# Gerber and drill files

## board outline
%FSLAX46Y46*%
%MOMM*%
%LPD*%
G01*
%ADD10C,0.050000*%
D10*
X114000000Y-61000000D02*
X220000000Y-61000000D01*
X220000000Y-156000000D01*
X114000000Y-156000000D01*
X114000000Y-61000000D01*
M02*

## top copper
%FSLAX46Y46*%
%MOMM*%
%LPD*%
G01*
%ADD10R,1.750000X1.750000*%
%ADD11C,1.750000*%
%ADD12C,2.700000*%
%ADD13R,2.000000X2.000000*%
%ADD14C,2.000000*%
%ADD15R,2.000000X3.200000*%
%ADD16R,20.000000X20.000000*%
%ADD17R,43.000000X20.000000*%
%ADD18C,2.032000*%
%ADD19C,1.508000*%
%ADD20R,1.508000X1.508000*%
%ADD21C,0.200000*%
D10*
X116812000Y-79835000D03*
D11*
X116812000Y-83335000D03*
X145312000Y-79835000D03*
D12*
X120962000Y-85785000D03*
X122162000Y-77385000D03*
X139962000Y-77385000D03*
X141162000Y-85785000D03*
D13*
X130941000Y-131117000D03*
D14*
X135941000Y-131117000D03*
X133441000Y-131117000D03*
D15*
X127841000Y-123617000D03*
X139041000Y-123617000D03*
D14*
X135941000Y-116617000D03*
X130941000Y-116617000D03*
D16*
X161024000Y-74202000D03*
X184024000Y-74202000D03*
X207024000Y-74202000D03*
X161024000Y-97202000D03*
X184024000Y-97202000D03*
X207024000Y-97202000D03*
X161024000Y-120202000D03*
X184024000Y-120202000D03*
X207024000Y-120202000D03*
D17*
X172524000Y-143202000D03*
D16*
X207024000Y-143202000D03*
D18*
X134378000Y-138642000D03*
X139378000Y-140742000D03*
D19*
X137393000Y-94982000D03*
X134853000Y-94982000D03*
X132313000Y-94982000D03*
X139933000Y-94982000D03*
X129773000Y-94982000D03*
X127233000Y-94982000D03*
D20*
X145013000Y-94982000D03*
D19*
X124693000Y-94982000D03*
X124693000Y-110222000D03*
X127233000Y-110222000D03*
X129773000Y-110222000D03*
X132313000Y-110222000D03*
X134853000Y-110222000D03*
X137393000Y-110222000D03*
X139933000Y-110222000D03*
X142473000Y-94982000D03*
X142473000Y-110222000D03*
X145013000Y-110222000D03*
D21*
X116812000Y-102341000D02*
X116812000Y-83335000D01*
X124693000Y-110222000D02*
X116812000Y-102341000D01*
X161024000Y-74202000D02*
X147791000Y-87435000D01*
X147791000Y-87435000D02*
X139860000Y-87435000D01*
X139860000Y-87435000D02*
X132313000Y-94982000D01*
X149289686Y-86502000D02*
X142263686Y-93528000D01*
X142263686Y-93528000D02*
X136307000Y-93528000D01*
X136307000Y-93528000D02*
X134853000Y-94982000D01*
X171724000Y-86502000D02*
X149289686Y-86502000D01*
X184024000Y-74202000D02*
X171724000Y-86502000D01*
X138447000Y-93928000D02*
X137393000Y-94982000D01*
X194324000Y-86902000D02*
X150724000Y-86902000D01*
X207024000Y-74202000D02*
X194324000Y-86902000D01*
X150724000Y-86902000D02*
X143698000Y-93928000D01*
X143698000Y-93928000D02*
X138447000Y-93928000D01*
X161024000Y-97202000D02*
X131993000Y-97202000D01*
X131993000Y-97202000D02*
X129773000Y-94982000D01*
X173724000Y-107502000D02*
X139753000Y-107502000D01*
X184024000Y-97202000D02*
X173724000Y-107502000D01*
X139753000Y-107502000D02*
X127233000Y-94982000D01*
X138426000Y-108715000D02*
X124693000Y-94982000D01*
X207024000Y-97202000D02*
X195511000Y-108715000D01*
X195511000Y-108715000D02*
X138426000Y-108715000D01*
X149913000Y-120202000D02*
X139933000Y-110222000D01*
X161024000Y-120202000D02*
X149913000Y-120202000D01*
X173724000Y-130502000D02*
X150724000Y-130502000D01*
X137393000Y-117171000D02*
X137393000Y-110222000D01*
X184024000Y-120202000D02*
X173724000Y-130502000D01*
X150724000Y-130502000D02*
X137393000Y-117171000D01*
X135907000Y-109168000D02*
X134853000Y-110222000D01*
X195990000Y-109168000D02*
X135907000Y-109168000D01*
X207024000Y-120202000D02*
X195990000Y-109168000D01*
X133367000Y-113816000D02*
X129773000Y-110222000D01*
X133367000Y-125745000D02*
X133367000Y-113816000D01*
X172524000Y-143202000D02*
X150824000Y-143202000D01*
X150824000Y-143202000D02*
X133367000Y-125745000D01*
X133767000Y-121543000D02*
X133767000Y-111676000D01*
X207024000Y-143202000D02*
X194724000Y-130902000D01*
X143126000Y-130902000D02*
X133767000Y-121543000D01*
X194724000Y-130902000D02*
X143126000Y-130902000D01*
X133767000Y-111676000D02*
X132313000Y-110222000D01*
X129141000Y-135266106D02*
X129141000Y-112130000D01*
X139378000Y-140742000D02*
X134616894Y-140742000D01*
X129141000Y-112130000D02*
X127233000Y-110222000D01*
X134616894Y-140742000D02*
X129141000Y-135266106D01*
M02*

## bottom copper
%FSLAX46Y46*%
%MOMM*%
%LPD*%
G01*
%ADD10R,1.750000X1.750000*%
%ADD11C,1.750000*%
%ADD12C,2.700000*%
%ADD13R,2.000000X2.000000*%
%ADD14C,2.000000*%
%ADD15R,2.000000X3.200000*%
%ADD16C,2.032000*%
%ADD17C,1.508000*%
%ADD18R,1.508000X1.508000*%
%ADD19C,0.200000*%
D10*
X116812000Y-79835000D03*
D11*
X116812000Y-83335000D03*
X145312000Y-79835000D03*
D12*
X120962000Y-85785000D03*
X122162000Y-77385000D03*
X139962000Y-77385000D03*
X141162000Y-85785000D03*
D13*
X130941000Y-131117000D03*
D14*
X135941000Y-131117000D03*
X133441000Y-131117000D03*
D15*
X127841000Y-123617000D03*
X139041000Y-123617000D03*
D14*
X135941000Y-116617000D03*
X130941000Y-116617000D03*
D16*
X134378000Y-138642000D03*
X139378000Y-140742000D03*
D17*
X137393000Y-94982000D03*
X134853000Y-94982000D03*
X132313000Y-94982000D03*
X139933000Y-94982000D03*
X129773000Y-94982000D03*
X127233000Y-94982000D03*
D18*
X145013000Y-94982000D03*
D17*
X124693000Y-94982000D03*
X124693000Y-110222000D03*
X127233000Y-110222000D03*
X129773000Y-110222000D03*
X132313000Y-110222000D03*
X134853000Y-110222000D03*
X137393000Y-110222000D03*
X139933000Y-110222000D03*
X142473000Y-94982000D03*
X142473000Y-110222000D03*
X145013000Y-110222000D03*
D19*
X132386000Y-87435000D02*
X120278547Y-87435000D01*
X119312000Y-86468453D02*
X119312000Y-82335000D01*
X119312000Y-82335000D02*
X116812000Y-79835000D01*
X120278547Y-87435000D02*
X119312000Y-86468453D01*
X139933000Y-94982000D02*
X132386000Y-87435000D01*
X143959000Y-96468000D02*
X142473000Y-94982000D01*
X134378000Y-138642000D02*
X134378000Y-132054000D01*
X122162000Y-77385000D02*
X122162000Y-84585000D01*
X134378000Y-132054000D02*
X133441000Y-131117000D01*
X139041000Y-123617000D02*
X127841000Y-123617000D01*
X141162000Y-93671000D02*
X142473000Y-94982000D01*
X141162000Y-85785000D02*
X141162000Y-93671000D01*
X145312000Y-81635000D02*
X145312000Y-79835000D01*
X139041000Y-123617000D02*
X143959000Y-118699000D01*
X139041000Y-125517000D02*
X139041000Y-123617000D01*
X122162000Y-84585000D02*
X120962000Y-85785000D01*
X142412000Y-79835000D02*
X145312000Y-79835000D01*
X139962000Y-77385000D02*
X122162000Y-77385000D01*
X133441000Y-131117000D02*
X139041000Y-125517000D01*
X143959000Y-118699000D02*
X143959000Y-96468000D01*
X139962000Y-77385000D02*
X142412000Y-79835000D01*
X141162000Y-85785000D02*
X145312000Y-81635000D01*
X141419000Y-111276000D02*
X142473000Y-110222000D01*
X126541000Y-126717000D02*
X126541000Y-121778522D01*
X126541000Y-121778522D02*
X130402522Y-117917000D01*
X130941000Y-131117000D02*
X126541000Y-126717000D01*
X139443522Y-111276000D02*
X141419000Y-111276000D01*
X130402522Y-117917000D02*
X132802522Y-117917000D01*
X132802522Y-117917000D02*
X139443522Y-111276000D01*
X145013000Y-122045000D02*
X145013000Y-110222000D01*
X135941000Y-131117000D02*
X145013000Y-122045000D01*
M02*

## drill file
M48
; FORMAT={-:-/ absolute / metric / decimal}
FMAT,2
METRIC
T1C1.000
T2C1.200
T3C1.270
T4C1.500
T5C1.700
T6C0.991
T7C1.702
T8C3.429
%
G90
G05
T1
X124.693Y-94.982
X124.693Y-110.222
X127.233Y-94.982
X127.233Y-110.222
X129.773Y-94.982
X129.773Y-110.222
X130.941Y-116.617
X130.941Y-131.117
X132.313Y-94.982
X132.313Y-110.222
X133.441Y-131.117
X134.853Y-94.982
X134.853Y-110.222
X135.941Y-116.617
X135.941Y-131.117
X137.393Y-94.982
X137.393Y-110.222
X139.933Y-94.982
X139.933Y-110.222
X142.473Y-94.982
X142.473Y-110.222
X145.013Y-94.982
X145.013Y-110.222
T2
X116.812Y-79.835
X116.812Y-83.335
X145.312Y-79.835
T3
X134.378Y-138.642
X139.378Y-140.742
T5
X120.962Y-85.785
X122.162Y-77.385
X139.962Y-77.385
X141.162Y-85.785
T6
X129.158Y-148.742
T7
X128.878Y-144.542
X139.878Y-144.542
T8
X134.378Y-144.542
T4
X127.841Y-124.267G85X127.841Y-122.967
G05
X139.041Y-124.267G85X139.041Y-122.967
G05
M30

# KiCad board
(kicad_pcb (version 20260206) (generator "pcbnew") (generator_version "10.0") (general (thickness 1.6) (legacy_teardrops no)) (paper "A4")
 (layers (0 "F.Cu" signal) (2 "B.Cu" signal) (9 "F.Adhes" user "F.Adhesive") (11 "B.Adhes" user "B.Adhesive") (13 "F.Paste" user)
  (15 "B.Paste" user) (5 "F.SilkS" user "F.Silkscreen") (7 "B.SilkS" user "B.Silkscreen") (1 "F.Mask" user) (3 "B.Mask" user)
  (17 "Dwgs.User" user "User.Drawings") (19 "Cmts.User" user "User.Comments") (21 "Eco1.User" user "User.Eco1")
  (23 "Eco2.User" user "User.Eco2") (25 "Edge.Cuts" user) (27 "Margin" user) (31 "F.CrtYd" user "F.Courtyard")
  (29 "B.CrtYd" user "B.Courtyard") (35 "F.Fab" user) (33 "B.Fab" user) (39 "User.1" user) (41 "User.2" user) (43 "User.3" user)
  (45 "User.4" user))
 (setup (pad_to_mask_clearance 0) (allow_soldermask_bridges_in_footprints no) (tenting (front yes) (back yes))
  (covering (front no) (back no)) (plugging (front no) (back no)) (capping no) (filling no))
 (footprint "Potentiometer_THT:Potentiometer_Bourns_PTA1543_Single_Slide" (layer "F.Cu") (at 116.812 79.835)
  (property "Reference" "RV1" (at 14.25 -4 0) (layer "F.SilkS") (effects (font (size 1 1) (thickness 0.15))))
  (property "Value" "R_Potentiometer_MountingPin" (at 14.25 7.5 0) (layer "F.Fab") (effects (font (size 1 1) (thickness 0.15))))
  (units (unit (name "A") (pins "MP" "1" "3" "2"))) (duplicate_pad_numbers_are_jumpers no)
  (pad "1" thru_hole rect (at 0 0) (size 1.75 1.75) (drill 1.2) (layers "*.Cu" "*.Mask") (remove_unused_layers no) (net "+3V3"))
  (pad "2" thru_hole circle (at 0 3.5) (size 1.75 1.75) (drill 1.2) (layers "*.Cu" "*.Mask") (remove_unused_layers no) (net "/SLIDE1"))
  (pad "3" thru_hole circle (at 28.5 0) (size 1.75 1.75) (drill 1.2) (layers "*.Cu" "*.Mask") (remove_unused_layers no) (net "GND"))
  (pad "MP" thru_hole circle (at 4.15 5.95) (size 2.7 2.7) (drill 1.7) (layers "*.Cu" "*.Mask") (remove_unused_layers no) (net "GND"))
  (pad "MP" thru_hole circle (at 5.35 -2.45) (size 2.7 2.7) (drill 1.7) (layers "*.Cu" "*.Mask") (remove_unused_layers no) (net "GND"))
  (pad "MP" thru_hole circle (at 23.15 -2.45) (size 2.7 2.7) (drill 1.7) (layers "*.Cu" "*.Mask") (remove_unused_layers no) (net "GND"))
  (pad "MP" thru_hole circle (at 24.35 5.95) (size 2.7 2.7) (drill 1.7) (layers "*.Cu" "*.Mask") (remove_unused_layers no) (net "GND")))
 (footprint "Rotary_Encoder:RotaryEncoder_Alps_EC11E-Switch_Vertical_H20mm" (layer "F.Cu") (at 130.941 131.117 90)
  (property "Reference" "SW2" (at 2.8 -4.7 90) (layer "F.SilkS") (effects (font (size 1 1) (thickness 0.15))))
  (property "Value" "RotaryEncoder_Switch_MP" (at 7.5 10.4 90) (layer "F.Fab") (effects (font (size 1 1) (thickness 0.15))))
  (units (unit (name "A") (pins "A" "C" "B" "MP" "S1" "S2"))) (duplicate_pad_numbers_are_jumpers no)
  (pad "A" thru_hole rect (at 0 0 90) (size 2 2) (drill 1) (layers "*.Cu" "*.Mask") (remove_unused_layers no) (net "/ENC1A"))
  (pad "B" thru_hole circle (at 0 5 90) (size 2 2) (drill 1) (layers "*.Cu" "*.Mask") (remove_unused_layers no) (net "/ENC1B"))
  (pad "C" thru_hole circle (at 0 2.5 90) (size 2 2) (drill 1) (layers "*.Cu" "*.Mask") (remove_unused_layers no) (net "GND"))
  (pad "MP" thru_hole rect (at 7.5 -3.1 90) (size 3.2 2) (drill oval 2.8 1.5) (layers "*.Cu" "*.Mask") (remove_unused_layers no) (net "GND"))
  (pad "MP" thru_hole rect (at 7.5 8.1 90) (size 3.2 2) (drill oval 2.8 1.5) (layers "*.Cu" "*.Mask") (remove_unused_layers no) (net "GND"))
  (pad "S1" thru_hole circle (at 14.5 5 90) (size 2 2) (drill 1) (layers "*.Cu" "*.Mask") (remove_unused_layers no)
   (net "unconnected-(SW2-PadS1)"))
  (pad "S2" thru_hole circle (at 14.5 0 90) (size 2 2) (drill 1) (layers "*.Cu" "*.Mask") (remove_unused_layers no)
   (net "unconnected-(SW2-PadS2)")))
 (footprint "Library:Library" (layer "F.Cu") (at 180.024 57.202)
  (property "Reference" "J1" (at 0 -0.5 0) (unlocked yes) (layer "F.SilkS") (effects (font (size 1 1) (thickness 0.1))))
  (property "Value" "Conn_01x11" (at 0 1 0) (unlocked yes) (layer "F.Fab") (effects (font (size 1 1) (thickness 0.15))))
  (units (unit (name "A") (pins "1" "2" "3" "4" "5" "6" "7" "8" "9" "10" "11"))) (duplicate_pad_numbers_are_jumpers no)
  (pad "1" smd rect (at -19 17) (size 20 20) (layers "F.Cu" "F.Mask") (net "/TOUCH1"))
  (pad "2" smd rect (at 4 17) (size 20 20) (layers "F.Cu" "F.Mask") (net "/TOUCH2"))
  (pad "3" smd rect (at 27 17) (size 20 20) (layers "F.Cu" "F.Mask") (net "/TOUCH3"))
  (pad "4" smd rect (at -19 40) (size 20 20) (layers "F.Cu" "F.Mask") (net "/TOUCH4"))
  (pad "5" smd rect (at 4 40) (size 20 20) (layers "F.Cu" "F.Mask") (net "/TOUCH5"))
  (pad "6" smd rect (at 27 40) (size 20 20) (layers "F.Cu" "F.Mask") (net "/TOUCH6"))
  (pad "7" smd rect (at -19 63) (size 20 20) (layers "F.Cu" "F.Mask") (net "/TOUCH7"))
  (pad "8" smd rect (at 4 63) (size 20 20) (layers "F.Cu" "F.Mask") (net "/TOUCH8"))
  (pad "9" smd rect (at 27 63) (size 20 20) (layers "F.Cu" "F.Mask") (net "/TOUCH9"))
  (pad "10" smd rect (at -7.5 86) (size 43 20) (layers "F.Cu" "F.Mask") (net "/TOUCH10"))
  (pad "11" smd rect (at 27 86) (size 20 20) (layers "F.Cu" "F.Mask") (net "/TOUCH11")))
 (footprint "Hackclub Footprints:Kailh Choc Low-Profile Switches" (layer "F.Cu") (at 134.378 144.542 180)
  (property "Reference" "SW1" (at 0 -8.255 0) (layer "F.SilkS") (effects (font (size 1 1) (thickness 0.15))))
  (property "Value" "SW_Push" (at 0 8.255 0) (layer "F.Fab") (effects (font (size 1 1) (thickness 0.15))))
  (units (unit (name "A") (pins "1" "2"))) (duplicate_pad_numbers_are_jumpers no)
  (pad "" np_thru_hole circle (at -5.5 0 180) (size 1.7018 1.7018) (drill 1.7018) (layers "*.Cu" "*.Mask"))
  (pad "" np_thru_hole circle (at 0 0 180) (size 3.429 3.429) (drill 3.429) (layers "*.Cu" "*.Mask"))
  (pad "" np_thru_hole circle (at 5.22 -4.2 180) (size 0.9906 0.9906) (drill 0.9906) (layers "*.Cu" "*.Mask"))
  (pad "" np_thru_hole circle (at 5.5 0 180) (size 1.7018 1.7018) (drill 1.7018) (layers "*.Cu" "*.Mask"))
  (pad "1" thru_hole circle (at 0 5.9 180) (size 2.032 2.032) (drill 1.27) (layers "*.Cu" "*.Mask") (remove_unused_layers no) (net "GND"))
  (pad "2" thru_hole circle (at -5 3.8 180) (size 2.032 2.032) (drill 1.27) (layers "*.Cu" "*.Mask") (remove_unused_layers no)
   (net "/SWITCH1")))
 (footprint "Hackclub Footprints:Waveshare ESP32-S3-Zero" (layer "F.Cu") (at 134.853 102.602 -90)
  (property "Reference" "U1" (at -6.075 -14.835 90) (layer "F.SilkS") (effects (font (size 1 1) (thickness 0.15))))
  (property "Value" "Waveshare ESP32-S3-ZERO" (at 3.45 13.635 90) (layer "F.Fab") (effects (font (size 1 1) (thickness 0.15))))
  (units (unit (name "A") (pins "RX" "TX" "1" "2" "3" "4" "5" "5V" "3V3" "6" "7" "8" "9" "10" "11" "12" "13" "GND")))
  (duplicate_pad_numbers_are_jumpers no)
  (pad "1" thru_hole circle (at -7.62 -2.54 270) (size 1.508 1.508) (drill 1) (layers "*.Cu" "*.Mask") (remove_unused_layers no)
   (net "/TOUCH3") (solder_mask_margin 0.102))
  (pad "2" thru_hole circle (at -7.62 0 270) (size 1.508 1.508) (drill 1) (layers "*.Cu" "*.Mask") (remove_unused_layers no) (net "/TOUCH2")
   (solder_mask_margin 0.102))
  (pad "3" thru_hole circle (at -7.62 2.54 270) (size 1.508 1.508) (drill 1) (layers "*.Cu" "*.Mask") (remove_unused_layers no)
   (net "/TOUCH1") (solder_mask_margin 0.102))
  (pad "3V3" thru_hole circle (at -7.62 -5.08 270) (size 1.508 1.508) (drill 1) (layers "*.Cu" "*.Mask") (remove_unused_layers no)
   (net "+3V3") (solder_mask_margin 0.102))
  (pad "4" thru_hole circle (at -7.62 5.08 270) (size 1.508 1.508) (drill 1) (layers "*.Cu" "*.Mask") (remove_unused_layers no)
   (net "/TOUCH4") (solder_mask_margin 0.102))
  (pad "5" thru_hole circle (at -7.62 7.62 270) (size 1.508 1.508) (drill 1) (layers "*.Cu" "*.Mask") (remove_unused_layers no)
   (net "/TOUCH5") (solder_mask_margin 0.102))
  (pad "5V" thru_hole rect (at -7.62 -10.16 270) (size 1.508 1.508) (drill 1) (layers "*.Cu" "*.Mask") (remove_unused_layers no) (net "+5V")
   (solder_mask_margin 0.102))
  (pad "6" thru_hole circle (at -7.62 10.16 270) (size 1.508 1.508) (drill 1) (layers "*.Cu" "*.Mask") (remove_unused_layers no)
   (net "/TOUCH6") (solder_mask_margin 0.102))
  (pad "7" thru_hole circle (at 7.62 10.16 270) (size 1.508 1.508) (drill 1) (layers "*.Cu" "*.Mask") (remove_unused_layers no)
   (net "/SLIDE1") (solder_mask_margin 0.102))
  (pad "8" thru_hole circle (at 7.62 7.62 270) (size 1.508 1.508) (drill 1) (layers "*.Cu" "*.Mask") (remove_unused_layers no)
   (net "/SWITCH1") (solder_mask_margin 0.102))
  (pad "9" thru_hole circle (at 7.62 5.08 270) (size 1.508 1.508) (drill 1) (layers "*.Cu" "*.Mask") (remove_unused_layers no)
   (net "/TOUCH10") (solder_mask_margin 0.102))
  (pad "10" thru_hole circle (at 7.62 2.54 270) (size 1.508 1.508) (drill 1) (layers "*.Cu" "*.Mask") (remove_unused_layers no)
   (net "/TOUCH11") (solder_mask_margin 0.102))
  (pad "11" thru_hole circle (at 7.62 0 270) (size 1.508 1.508) (drill 1) (layers "*.Cu" "*.Mask") (remove_unused_layers no) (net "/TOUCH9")
   (solder_mask_margin 0.102))
  (pad "12" thru_hole circle (at 7.62 -2.54 270) (size 1.508 1.508) (drill 1) (layers "*.Cu" "*.Mask") (remove_unused_layers no)
   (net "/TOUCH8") (solder_mask_margin 0.102))
  (pad "13" thru_hole circle (at 7.62 -5.08 270) (size 1.508 1.508) (drill 1) (layers "*.Cu" "*.Mask") (remove_unused_layers no)
   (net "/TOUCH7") (solder_mask_margin 0.102))
  (pad "GND" thru_hole circle (at -7.62 -7.62 270) (size 1.508 1.508) (drill 1) (layers "*.Cu" "*.Mask") (remove_unused_layers no)
   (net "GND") (solder_mask_margin 0.102))
  (pad "RX" thru_hole circle (at 7.62 -7.62 270) (size 1.508 1.508) (drill 1) (layers "*.Cu" "*.Mask") (remove_unused_layers no)
   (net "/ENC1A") (solder_mask_margin 0.102))
  (pad "TX" thru_hole circle (at 7.62 -10.16 270) (size 1.508 1.508) (drill 1) (layers "*.Cu" "*.Mask") (remove_unused_layers no)
   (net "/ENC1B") (solder_mask_margin 0.102)))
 (gr_rect (start 114 61) (end 220 156) (stroke (width 0.05) (type default)) (fill no) (layer "Edge.Cuts"))
 (segment (start 132.386 87.435) (end 120.278547 87.435) (width 0.2) (layer "B.Cu") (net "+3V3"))
 (segment (start 119.312 86.468453) (end 119.312 82.335) (width 0.2) (layer "B.Cu") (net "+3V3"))
 (segment (start 119.312 82.335) (end 116.812 79.835) (width 0.2) (layer "B.Cu") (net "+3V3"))
 (segment (start 120.278547 87.435) (end 119.312 86.468453) (width 0.2) (layer "B.Cu") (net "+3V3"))
 (segment (start 139.933 94.982) (end 132.386 87.435) (width 0.2) (layer "B.Cu") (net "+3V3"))
 (segment (start 116.812 102.341) (end 116.812 83.335) (width 0.2) (layer "F.Cu") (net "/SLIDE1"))
 (segment (start 124.693 110.222) (end 116.812 102.341) (width 0.2) (layer "F.Cu") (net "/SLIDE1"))
 (segment (start 143.959 96.468) (end 142.473 94.982) (width 0.2) (layer "B.Cu") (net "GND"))
 (segment (start 134.378 138.642) (end 134.378 132.054) (width 0.2) (layer "B.Cu") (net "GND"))
 (segment (start 122.162 77.385) (end 122.162 84.585) (width 0.2) (layer "B.Cu") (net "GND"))
 (segment (start 134.378 132.054) (end 133.441 131.117) (width 0.2) (layer "B.Cu") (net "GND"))
 (segment (start 139.041 123.617) (end 127.841 123.617) (width 0.2) (layer "B.Cu") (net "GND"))
 (segment (start 141.162 93.671) (end 142.473 94.982) (width 0.2) (layer "B.Cu") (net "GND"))
 (segment (start 141.162 85.785) (end 141.162 93.671) (width 0.2) (layer "B.Cu") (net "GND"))
 (segment (start 145.312 81.635) (end 145.312 79.835) (width 0.2) (layer "B.Cu") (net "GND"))
 (segment (start 139.041 123.617) (end 143.959 118.699) (width 0.2) (layer "B.Cu") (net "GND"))
 (segment (start 139.041 125.517) (end 139.041 123.617) (width 0.2) (layer "B.Cu") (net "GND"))
 (segment (start 122.162 84.585) (end 120.962 85.785) (width 0.2) (layer "B.Cu") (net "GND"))
 (segment (start 142.412 79.835) (end 145.312 79.835) (width 0.2) (layer "B.Cu") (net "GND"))
 (segment (start 139.962 77.385) (end 122.162 77.385) (width 0.2) (layer "B.Cu") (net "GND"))
 (segment (start 133.441 131.117) (end 139.041 125.517) (width 0.2) (layer "B.Cu") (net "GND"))
 (segment (start 143.959 118.699) (end 143.959 96.468) (width 0.2) (layer "B.Cu") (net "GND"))
 (segment (start 139.962 77.385) (end 142.412 79.835) (width 0.2) (layer "B.Cu") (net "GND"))
 (segment (start 141.162 85.785) (end 145.312 81.635) (width 0.2) (layer "B.Cu") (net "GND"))
 (segment (start 141.419 111.276) (end 142.473 110.222) (width 0.2) (layer "B.Cu") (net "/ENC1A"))
 (segment (start 126.541 126.717) (end 126.541 121.778522) (width 0.2) (layer "B.Cu") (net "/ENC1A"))
 (segment (start 126.541 121.778522) (end 130.402522 117.917) (width 0.2) (layer "B.Cu") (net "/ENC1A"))
 (segment (start 130.941 131.117) (end 126.541 126.717) (width 0.2) (layer "B.Cu") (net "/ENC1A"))
 (segment (start 139.443522 111.276) (end 141.419 111.276) (width 0.2) (layer "B.Cu") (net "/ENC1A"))
 (segment (start 130.402522 117.917) (end 132.802522 117.917) (width 0.2) (layer "B.Cu") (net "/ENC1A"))
 (segment (start 132.802522 117.917) (end 139.443522 111.276) (width 0.2) (layer "B.Cu") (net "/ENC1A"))
 (segment (start 145.013 122.045) (end 145.013 110.222) (width 0.2) (layer "B.Cu") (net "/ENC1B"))
 (segment (start 135.941 131.117) (end 145.013 122.045) (width 0.2) (layer "B.Cu") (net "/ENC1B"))
 (segment (start 161.024 74.202) (end 147.791 87.435) (width 0.2) (layer "F.Cu") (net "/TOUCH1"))
 (segment (start 147.791 87.435) (end 139.86 87.435) (width 0.2) (layer "F.Cu") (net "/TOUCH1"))
 (segment (start 139.86 87.435) (end 132.313 94.982) (width 0.2) (layer "F.Cu") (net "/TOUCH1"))
 (segment (start 149.289686 86.502) (end 142.263686 93.528) (width 0.2) (layer "F.Cu") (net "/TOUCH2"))
 (segment (start 142.263686 93.528) (end 136.307 93.528) (width 0.2) (layer "F.Cu") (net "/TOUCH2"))
 (segment (start 136.307 93.528) (end 134.853 94.982) (width 0.2) (layer "F.Cu") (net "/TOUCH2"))
 (segment (start 171.724 86.502) (end 149.289686 86.502) (width 0.2) (layer "F.Cu") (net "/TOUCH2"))
 (segment (start 184.024 74.202) (end 171.724 86.502) (width 0.2) (layer "F.Cu") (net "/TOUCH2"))
 (segment (start 138.447 93.928) (end 137.393 94.982) (width 0.2) (layer "F.Cu") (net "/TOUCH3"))
 (segment (start 194.324 86.902) (end 150.724 86.902) (width 0.2) (layer "F.Cu") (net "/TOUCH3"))
 (segment (start 207.024 74.202) (end 194.324 86.902) (width 0.2) (layer "F.Cu") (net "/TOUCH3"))
 (segment (start 150.724 86.902) (end 143.698 93.928) (width 0.2) (layer "F.Cu") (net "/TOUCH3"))
 (segment (start 143.698 93.928) (end 138.447 93.928) (width 0.2) (layer "F.Cu") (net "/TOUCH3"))
 (segment (start 161.024 97.202) (end 131.993 97.202) (width 0.2) (layer "F.Cu") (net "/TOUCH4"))
 (segment (start 131.993 97.202) (end 129.773 94.982) (width 0.2) (layer "F.Cu") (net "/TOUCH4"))
 (segment (start 173.724 107.502) (end 139.753 107.502) (width 0.2) (layer "F.Cu") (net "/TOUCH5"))
 (segment (start 184.024 97.202) (end 173.724 107.502) (width 0.2) (layer "F.Cu") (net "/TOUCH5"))
 (segment (start 139.753 107.502) (end 127.233 94.982) (width 0.2) (layer "F.Cu") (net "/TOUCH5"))
 (segment (start 138.426 108.715) (end 124.693 94.982) (width 0.2) (layer "F.Cu") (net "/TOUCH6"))
 (segment (start 207.024 97.202) (end 195.511 108.715) (width 0.2) (layer "F.Cu") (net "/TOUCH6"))
 (segment (start 195.511 108.715) (end 138.426 108.715) (width 0.2) (layer "F.Cu") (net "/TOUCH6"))
 (segment (start 149.913 120.202) (end 139.933 110.222) (width 0.2) (layer "F.Cu") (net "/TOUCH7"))
 (segment (start 161.024 120.202) (end 149.913 120.202) (width 0.2) (layer "F.Cu") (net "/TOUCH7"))
 (segment (start 173.724 130.502) (end 150.724 130.502) (width 0.2) (layer "F.Cu") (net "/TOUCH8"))
 (segment (start 137.393 117.171) (end 137.393 110.222) (width 0.2) (layer "F.Cu") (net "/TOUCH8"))
 (segment (start 184.024 120.202) (end 173.724 130.502) (width 0.2) (layer "F.Cu") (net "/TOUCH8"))
 (segment (start 150.724 130.502) (end 137.393 117.171) (width 0.2) (layer "F.Cu") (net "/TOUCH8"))
 (segment (start 135.907 109.168) (end 134.853 110.222) (width 0.2) (layer "F.Cu") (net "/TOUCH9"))
 (segment (start 195.99 109.168) (end 135.907 109.168) (width 0.2) (layer "F.Cu") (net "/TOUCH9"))
 (segment (start 207.024 120.202) (end 195.99 109.168) (width 0.2) (layer "F.Cu") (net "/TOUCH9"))
 (segment (start 133.367 113.816) (end 129.773 110.222) (width 0.2) (layer "F.Cu") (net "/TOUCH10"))
 (segment (start 133.367 125.745) (end 133.367 113.816) (width 0.2) (layer "F.Cu") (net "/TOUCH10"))
 (segment (start 172.524 143.202) (end 150.824 143.202) (width 0.2) (layer "F.Cu") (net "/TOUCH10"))
 (segment (start 150.824 143.202) (end 133.367 125.745) (width 0.2) (layer "F.Cu") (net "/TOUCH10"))
 (segment (start 133.767 121.543) (end 133.767 111.676) (width 0.2) (layer "F.Cu") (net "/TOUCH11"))
 (segment (start 207.024 143.202) (end 194.724 130.902) (width 0.2) (layer "F.Cu") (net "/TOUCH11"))
 (segment (start 143.126 130.902) (end 133.767 121.543) (width 0.2) (layer "F.Cu") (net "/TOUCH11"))
 (segment (start 194.724 130.902) (end 143.126 130.902) (width 0.2) (layer "F.Cu") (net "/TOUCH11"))
 (segment (start 133.767 111.676) (end 132.313 110.222) (width 0.2) (layer "F.Cu") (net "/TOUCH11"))
 (segment (start 129.141 135.266106) (end 129.141 112.13) (width 0.2) (layer "F.Cu") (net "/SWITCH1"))
 (segment (start 139.378 140.742) (end 134.616894 140.742) (width 0.2) (layer "F.Cu") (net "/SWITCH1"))
 (segment (start 129.141 112.13) (end 127.233 110.222) (width 0.2) (layer "F.Cu") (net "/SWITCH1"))
 (segment (start 134.616894 140.742) (end 129.141 135.266106) (width 0.2) (layer "F.Cu") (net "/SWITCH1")))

